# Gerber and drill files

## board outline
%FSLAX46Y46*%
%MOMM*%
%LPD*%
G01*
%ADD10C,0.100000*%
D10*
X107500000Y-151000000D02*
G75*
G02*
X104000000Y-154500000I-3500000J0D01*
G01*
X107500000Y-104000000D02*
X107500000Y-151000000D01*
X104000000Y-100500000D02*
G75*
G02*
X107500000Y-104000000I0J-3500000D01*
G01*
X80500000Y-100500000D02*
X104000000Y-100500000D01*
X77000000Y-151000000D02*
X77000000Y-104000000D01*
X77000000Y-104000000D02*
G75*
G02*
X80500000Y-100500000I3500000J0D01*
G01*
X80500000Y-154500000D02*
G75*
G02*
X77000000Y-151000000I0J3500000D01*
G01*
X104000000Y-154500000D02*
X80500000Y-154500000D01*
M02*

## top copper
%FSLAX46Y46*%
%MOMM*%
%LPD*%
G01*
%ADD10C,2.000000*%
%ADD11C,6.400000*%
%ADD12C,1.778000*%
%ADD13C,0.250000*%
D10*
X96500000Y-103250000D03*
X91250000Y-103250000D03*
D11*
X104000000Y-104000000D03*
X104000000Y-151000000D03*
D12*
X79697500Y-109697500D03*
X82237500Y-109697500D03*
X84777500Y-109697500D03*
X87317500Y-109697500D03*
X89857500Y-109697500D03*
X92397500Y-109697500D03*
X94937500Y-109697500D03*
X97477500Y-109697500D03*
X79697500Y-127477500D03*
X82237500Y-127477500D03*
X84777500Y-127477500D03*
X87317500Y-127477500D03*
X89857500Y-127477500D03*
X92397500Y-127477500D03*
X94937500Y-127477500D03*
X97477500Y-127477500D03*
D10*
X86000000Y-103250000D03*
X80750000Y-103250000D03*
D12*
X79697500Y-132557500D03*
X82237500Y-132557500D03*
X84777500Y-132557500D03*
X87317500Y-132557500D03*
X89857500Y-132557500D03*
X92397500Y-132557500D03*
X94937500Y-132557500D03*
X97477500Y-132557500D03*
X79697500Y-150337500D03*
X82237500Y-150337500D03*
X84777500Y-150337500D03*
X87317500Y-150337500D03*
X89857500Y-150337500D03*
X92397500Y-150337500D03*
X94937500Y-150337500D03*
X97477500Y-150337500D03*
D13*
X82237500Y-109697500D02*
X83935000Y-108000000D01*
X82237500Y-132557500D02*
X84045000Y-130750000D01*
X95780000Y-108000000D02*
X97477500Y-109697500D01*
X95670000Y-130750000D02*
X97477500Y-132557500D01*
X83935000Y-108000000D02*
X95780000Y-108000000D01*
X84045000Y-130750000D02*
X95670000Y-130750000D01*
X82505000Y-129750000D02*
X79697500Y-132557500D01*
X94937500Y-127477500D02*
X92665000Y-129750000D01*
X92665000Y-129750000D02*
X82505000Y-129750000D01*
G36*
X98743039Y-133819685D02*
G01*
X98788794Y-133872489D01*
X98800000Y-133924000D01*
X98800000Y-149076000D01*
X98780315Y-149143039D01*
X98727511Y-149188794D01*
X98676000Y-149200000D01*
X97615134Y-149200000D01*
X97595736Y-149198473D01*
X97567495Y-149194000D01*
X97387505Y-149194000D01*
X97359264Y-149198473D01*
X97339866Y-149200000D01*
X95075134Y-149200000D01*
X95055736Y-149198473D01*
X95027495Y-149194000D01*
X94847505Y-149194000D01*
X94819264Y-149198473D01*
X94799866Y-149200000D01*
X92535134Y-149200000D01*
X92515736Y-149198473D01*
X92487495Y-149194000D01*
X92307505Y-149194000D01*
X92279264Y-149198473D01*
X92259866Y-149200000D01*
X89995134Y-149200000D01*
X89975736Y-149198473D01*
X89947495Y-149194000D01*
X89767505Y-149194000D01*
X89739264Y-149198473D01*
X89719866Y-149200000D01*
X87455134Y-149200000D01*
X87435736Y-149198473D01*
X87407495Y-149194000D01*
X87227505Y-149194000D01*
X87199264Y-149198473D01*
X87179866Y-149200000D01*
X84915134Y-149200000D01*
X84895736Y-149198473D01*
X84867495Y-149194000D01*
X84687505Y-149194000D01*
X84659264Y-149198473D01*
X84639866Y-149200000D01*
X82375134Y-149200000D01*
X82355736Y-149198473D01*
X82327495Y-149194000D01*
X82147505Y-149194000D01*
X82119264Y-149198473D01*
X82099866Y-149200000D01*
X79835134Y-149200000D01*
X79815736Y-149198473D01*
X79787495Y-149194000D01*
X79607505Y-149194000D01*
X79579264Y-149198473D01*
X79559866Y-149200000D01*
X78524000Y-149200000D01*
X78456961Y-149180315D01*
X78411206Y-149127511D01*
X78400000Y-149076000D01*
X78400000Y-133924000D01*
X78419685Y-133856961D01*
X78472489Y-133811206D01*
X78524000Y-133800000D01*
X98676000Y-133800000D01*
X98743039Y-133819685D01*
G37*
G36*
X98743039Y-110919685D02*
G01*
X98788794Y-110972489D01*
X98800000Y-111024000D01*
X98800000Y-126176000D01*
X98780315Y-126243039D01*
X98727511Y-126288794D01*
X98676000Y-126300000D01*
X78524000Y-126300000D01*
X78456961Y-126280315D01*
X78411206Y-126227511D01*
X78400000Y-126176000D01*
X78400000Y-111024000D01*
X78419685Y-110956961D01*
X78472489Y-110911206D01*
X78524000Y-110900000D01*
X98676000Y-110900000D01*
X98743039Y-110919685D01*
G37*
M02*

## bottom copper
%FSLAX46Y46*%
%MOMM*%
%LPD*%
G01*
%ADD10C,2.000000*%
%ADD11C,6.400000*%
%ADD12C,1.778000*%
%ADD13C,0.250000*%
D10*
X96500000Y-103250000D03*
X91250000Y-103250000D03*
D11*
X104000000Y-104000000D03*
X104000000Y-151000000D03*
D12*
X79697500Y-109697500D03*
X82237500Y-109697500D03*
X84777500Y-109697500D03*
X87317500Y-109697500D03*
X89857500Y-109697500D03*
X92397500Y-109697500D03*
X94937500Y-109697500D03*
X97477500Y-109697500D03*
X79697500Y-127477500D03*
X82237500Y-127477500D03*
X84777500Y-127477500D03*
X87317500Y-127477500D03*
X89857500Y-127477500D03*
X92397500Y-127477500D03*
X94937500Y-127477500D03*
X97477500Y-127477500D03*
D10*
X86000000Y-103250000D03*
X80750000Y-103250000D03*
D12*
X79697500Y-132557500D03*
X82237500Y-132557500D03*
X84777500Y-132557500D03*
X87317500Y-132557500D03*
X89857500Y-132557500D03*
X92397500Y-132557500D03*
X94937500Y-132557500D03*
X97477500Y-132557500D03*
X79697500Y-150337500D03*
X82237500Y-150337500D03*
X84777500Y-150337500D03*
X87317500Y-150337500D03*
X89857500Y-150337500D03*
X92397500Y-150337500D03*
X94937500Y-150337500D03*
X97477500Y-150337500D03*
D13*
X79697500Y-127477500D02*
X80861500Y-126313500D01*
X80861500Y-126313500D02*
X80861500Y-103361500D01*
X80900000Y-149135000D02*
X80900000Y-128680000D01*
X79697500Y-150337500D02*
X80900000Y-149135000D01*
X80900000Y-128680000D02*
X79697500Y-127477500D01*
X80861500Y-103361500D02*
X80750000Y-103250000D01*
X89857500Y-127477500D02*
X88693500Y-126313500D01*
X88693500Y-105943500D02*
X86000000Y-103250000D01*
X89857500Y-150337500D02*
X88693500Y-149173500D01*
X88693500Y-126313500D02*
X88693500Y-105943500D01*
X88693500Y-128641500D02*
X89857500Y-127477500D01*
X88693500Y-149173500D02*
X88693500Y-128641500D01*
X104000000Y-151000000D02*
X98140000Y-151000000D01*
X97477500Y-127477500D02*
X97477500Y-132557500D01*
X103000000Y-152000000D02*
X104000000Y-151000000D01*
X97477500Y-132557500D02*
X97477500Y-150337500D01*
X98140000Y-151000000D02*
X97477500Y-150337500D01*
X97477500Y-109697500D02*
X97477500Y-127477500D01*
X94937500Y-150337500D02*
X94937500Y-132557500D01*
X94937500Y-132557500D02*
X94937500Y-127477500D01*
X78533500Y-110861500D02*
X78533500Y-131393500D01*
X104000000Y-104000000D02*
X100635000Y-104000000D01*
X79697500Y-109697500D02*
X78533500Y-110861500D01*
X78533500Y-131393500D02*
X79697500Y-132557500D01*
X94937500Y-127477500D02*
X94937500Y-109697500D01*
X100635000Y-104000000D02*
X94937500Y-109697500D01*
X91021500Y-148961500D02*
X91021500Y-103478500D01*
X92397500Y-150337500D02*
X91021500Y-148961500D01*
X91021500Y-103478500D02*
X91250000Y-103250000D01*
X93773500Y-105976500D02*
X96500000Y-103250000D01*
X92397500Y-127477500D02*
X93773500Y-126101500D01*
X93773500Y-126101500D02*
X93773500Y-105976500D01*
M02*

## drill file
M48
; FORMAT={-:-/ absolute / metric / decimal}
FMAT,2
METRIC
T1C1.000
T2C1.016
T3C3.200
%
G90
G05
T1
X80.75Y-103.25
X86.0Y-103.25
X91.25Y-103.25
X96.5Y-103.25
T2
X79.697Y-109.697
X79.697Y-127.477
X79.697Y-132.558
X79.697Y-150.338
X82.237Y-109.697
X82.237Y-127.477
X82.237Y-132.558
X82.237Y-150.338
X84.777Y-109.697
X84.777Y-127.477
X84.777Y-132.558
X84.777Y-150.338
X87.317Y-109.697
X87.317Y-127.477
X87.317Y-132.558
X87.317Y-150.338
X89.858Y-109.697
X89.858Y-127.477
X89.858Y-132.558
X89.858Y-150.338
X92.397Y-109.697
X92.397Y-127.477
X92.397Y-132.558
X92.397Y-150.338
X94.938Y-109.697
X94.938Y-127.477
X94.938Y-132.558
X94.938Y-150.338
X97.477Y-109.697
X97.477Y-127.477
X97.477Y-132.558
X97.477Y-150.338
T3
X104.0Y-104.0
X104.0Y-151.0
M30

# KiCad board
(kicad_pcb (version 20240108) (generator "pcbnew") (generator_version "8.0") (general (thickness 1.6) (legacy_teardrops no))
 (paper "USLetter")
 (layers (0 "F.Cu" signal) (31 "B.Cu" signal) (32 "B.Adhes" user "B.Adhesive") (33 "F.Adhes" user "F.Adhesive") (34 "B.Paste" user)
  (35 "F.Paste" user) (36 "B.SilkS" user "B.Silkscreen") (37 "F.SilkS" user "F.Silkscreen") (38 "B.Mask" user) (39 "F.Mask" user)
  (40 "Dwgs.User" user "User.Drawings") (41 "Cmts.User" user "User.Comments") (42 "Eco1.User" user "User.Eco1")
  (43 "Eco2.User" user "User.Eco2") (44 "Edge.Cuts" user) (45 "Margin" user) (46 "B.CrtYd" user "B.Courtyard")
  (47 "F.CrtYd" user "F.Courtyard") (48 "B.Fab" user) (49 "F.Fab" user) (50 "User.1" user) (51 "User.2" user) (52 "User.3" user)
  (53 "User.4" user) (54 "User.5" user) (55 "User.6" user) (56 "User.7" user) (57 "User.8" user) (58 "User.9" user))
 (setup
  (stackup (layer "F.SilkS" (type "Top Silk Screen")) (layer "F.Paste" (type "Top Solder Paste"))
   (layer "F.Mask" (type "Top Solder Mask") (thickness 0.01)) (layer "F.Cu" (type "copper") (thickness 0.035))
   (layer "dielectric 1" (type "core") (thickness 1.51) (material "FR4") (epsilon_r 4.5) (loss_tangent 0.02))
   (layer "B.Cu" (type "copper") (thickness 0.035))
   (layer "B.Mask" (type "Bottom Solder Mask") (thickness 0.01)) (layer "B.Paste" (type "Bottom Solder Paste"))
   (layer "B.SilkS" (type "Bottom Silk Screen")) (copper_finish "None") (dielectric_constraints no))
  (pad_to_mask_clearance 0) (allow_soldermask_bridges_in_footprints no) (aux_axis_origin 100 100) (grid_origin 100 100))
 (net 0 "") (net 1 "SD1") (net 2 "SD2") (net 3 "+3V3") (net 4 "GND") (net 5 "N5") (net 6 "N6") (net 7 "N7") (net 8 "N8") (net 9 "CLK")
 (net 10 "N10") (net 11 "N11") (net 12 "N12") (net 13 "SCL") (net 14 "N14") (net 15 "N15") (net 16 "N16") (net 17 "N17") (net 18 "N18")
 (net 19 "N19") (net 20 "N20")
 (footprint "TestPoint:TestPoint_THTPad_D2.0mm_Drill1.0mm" (layer "F.Cu") (at 96.5 103.25)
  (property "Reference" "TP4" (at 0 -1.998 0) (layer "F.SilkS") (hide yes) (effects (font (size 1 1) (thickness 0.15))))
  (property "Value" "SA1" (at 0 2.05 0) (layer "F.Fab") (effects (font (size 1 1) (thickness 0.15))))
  (pad "1" thru_hole circle (at 0 0) (size 2 2) (drill 1) (layers "*.Cu" "*.Mask") (remove_unused_layers no) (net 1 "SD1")))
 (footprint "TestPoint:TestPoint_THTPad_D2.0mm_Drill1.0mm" (layer "F.Cu") (at 91.25 103.25)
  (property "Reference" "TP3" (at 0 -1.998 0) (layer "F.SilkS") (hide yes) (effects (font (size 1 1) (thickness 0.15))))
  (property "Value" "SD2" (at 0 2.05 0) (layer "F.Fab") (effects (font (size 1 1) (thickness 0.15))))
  (pad "1" thru_hole circle (at 0 0) (size 2 2) (drill 1) (layers "*.Cu" "*.Mask") (remove_unused_layers no) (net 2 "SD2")))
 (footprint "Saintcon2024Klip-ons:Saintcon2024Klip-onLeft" (layer "F.Cu") (at 139.75 126.4)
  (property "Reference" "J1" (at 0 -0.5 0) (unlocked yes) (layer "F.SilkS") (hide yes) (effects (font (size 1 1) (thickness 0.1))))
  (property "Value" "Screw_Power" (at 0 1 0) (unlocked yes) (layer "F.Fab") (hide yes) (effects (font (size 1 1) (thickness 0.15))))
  (pad "+" thru_hole circle (at -35.75 -22.4) (size 6.4 6.4) (drill 3.2) (layers "*.Cu" "*.Mask") (remove_unused_layers no) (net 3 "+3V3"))
  (pad "-" thru_hole circle (at -35.75 24.6) (size 6.4 6.4) (drill 3.2) (layers "*.Cu" "*.Mask") (remove_unused_layers no) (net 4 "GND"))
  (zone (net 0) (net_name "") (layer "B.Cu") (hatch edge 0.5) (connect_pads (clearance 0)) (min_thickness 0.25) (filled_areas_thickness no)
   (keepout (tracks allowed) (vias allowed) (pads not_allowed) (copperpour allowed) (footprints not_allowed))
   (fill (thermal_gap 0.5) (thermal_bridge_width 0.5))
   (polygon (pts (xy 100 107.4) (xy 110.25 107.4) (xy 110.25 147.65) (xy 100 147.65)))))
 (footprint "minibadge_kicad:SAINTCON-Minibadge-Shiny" (layer "F.Cu") (at 78.4275 108.4275)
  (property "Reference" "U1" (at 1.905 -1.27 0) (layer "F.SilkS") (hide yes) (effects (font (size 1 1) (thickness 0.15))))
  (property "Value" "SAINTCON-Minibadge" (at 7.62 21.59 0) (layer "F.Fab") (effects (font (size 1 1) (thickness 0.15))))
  (pad "1" thru_hole circle (at 1.27 1.27 90) (size 1.778 1.778) (drill 1.016) (layers "*.Cu" "*.Mask") (remove_unused_layers no)
   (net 3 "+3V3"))
  (pad "2" thru_hole circle (at 3.81 1.27 90) (size 1.778 1.778) (drill 1.016) (layers "*.Cu" "*.Mask") (remove_unused_layers no)
   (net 4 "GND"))
  (pad "3" thru_hole circle (at 6.35 1.27 90) (size 1.778 1.778) (drill 1.016) (layers "*.Cu" "*.Mask") (remove_unused_layers no)
   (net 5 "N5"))
  (pad "4" thru_hole circle (at 8.89 1.27 90) (size 1.778 1.778) (drill 1.016) (layers "*.Cu" "*.Mask") (remove_unused_layers no)
   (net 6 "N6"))
  (pad "5" thru_hole circle (at 11.43 1.27 90) (size 1.778 1.778) (drill 1.016) (layers "*.Cu" "*.Mask") (remove_unused_layers no)
   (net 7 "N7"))
  (pad "6" thru_hole circle (at 13.97 1.27 90) (size 1.778 1.778) (drill 1.016) (layers "*.Cu" "*.Mask") (remove_unused_layers no)
   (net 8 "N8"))
  (pad "7" thru_hole circle (at 16.51 1.27 90) (size 1.778 1.778) (drill 1.016) (layers "*.Cu" "*.Mask") (remove_unused_layers no)
   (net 3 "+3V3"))
  (pad "8" thru_hole circle (at 19.05 1.27 90) (size 1.778 1.778) (drill 1.016) (layers "*.Cu" "*.Mask") (remove_unused_layers no)
   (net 4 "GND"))
  (pad "9" thru_hole circle (at 1.27 19.05 90) (size 1.778 1.778) (drill 1.016) (layers "*.Cu" "*.Mask") (remove_unused_layers no)
   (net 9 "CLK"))
  (pad "10" thru_hole circle (at 3.81 19.05 90) (size 1.778 1.778) (drill 1.016) (layers "*.Cu" "*.Mask") (remove_unused_layers no)
   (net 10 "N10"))
  (pad "11" thru_hole circle (at 6.35 19.05 90) (size 1.778 1.778) (drill 1.016) (layers "*.Cu" "*.Mask") (remove_unused_layers no)
   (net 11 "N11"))
  (pad "12" thru_hole circle (at 8.89 19.05 90) (size 1.778 1.778) (drill 1.016) (layers "*.Cu" "*.Mask") (remove_unused_layers no)
   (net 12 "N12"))
  (pad "13" thru_hole circle (at 11.43 19.05 90) (size 1.778 1.778) (drill 1.016) (layers "*.Cu" "*.Mask") (remove_unused_layers no)
   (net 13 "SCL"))
  (pad "14" thru_hole circle (at 13.97 19.05 90) (size 1.778 1.778) (drill 1.016) (layers "*.Cu" "*.Mask") (remove_unused_layers no)
   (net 1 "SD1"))
  (pad "15" thru_hole circle (at 16.51 19.05 90) (size 1.778 1.778) (drill 1.016) (layers "*.Cu" "*.Mask") (remove_unused_layers no)
   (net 3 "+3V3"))
  (pad "16" thru_hole circle (at 19.05 19.05 90) (size 1.778 1.778) (drill 1.016) (layers "*.Cu" "*.Mask") (remove_unused_layers no)
   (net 4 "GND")))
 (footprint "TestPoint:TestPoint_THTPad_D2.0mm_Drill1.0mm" (layer "F.Cu") (at 86 103.25)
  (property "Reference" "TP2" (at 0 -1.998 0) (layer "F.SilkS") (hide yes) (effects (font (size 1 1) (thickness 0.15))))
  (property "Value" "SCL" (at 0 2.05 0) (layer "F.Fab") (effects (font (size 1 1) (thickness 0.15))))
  (pad "1" thru_hole circle (at 0 0) (size 2 2) (drill 1) (layers "*.Cu" "*.Mask") (remove_unused_layers no) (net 13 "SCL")))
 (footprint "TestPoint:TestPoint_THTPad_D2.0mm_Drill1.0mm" (layer "F.Cu") (at 80.75 103.25)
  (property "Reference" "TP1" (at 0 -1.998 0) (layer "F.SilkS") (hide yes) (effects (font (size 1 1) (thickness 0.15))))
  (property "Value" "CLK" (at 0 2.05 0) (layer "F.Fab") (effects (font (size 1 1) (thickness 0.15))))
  (pad "1" thru_hole circle (at 0 0) (size 2 2) (drill 1) (layers "*.Cu" "*.Mask") (remove_unused_layers no) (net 9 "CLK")))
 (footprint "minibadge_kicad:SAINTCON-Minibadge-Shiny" (layer "F.Cu") (at 78.4275 131.2875)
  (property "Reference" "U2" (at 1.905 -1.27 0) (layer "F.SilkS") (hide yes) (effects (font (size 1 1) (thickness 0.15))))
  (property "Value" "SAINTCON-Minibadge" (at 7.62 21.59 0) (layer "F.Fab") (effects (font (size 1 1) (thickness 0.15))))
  (pad "1" thru_hole circle (at 1.27 1.27 90) (size 1.778 1.778) (drill 1.016) (layers "*.Cu" "*.Mask") (remove_unused_layers no)
   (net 3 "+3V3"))
  (pad "2" thru_hole circle (at 3.81 1.27 90) (size 1.778 1.778) (drill 1.016) (layers "*.Cu" "*.Mask") (remove_unused_layers no)
   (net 4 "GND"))
  (pad "3" thru_hole circle (at 6.35 1.27 90) (size 1.778 1.778) (drill 1.016) (layers "*.Cu" "*.Mask") (remove_unused_layers no)
   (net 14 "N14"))
  (pad "4" thru_hole circle (at 8.89 1.27 90) (size 1.778 1.778) (drill 1.016) (layers "*.Cu" "*.Mask") (remove_unused_layers no)
   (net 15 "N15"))
  (pad "5" thru_hole circle (at 11.43 1.27 90) (size 1.778 1.778) (drill 1.016) (layers "*.Cu" "*.Mask") (remove_unused_layers no)
   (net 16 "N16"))
  (pad "6" thru_hole circle (at 13.97 1.27 90) (size 1.778 1.778) (drill 1.016) (layers "*.Cu" "*.Mask") (remove_unused_layers no)
   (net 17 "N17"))
  (pad "7" thru_hole circle (at 16.51 1.27 90) (size 1.778 1.778) (drill 1.016) (layers "*.Cu" "*.Mask") (remove_unused_layers no)
   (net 3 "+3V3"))
  (pad "8" thru_hole circle (at 19.05 1.27 90) (size 1.778 1.778) (drill 1.016) (layers "*.Cu" "*.Mask") (remove_unused_layers no)
   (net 4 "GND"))
  (pad "9" thru_hole circle (at 1.27 19.05 90) (size 1.778 1.778) (drill 1.016) (layers "*.Cu" "*.Mask") (remove_unused_layers no)
   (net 9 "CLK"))
  (pad "10" thru_hole circle (at 3.81 19.05 90) (size 1.778 1.778) (drill 1.016) (layers "*.Cu" "*.Mask") (remove_unused_layers no)
   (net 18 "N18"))
  (pad "11" thru_hole circle (at 6.35 19.05 90) (size 1.778 1.778) (drill 1.016) (layers "*.Cu" "*.Mask") (remove_unused_layers no)
   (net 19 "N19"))
  (pad "12" thru_hole circle (at 8.89 19.05 90) (size 1.778 1.778) (drill 1.016) (layers "*.Cu" "*.Mask") (remove_unused_layers no)
   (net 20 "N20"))
  (pad "13" thru_hole circle (at 11.43 19.05 90) (size 1.778 1.778) (drill 1.016) (layers "*.Cu" "*.Mask") (remove_unused_layers no)
   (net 13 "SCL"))
  (pad "14" thru_hole circle (at 13.97 19.05 90) (size 1.778 1.778) (drill 1.016) (layers "*.Cu" "*.Mask") (remove_unused_layers no)
   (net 2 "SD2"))
  (pad "15" thru_hole circle (at 16.51 19.05 90) (size 1.778 1.778) (drill 1.016) (layers "*.Cu" "*.Mask") (remove_unused_layers no)
   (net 3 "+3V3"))
  (pad "16" thru_hole circle (at 19.05 19.05 90) (size 1.778 1.778) (drill 1.016) (layers "*.Cu" "*.Mask") (remove_unused_layers no)
   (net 4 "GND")))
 (gr_arc (start 107.5 151) (mid 106.474874 153.474874) (end 104 154.5) (stroke (width 0.1) (type default)) (layer "Edge.Cuts"))
 (gr_line (start 107.5 104) (end 107.5 151) (stroke (width 0.1) (type default)) (layer "Edge.Cuts"))
 (gr_arc (start 104 100.5) (mid 106.474874 101.525126) (end 107.5 104) (stroke (width 0.1) (type default)) (layer "Edge.Cuts"))
 (gr_line (start 80.5 100.5) (end 104 100.5) (stroke (width 0.1) (type default)) (layer "Edge.Cuts"))
 (gr_line (start 77 151) (end 77 104) (stroke (width 0.1) (type default)) (layer "Edge.Cuts"))
 (gr_arc (start 77 104) (mid 78.025126 101.525126) (end 80.5 100.5) (stroke (width 0.1) (type default)) (layer "Edge.Cuts"))
 (gr_arc (start 80.5 154.5) (mid 78.025126 153.474874) (end 77 151) (stroke (width 0.1) (type default)) (layer "Edge.Cuts"))
 (gr_line (start 104 154.5) (end 80.5 154.5) (stroke (width 0.1) (type default)) (layer "Edge.Cuts"))
 (segment (start 79.6975 127.4775) (end 80.8615 126.3135) (width 0.25) (layer "B.Cu") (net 9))
 (segment (start 80.8615 126.3135) (end 80.8615 103.3615) (width 0.25) (layer "B.Cu") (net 9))
 (segment (start 80.9 149.135) (end 80.9 128.68) (width 0.25) (layer "B.Cu") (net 9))
 (segment (start 79.6975 150.3375) (end 80.9 149.135) (width 0.25) (layer "B.Cu") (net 9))
 (segment (start 80.9 128.68) (end 79.6975 127.4775) (width 0.25) (layer "B.Cu") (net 9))
 (segment (start 80.8615 103.3615) (end 80.75 103.25) (width 0.25) (layer "B.Cu") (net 9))
 (segment (start 89.8575 127.4775) (end 88.6935 126.3135) (width 0.25) (layer "B.Cu") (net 13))
 (segment (start 88.6935 105.9435) (end 86 103.25) (width 0.25) (layer "B.Cu") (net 13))
 (segment (start 89.8575 150.3375) (end 88.6935 149.1735) (width 0.25) (layer "B.Cu") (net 13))
 (segment (start 88.6935 126.3135) (end 88.6935 105.9435) (width 0.25) (layer "B.Cu") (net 13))
 (segment (start 88.6935 128.6415) (end 89.8575 127.4775) (width 0.25) (layer "B.Cu") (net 13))
 (segment (start 88.6935 149.1735) (end 88.6935 128.6415) (width 0.25) (layer "B.Cu") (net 13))
 (segment (start 82.2375 109.6975) (end 83.935 108) (width 0.25) (layer "F.Cu") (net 4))
 (segment (start 82.2375 132.5575) (end 84.045 130.75) (width 0.25) (layer "F.Cu") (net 4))
 (segment (start 95.78 108) (end 97.4775 109.6975) (width 0.25) (layer "F.Cu") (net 4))
 (segment (start 95.67 130.75) (end 97.4775 132.5575) (width 0.25) (layer "F.Cu") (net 4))
 (segment (start 83.935 108) (end 95.78 108) (width 0.25) (layer "F.Cu") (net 4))
 (segment (start 84.045 130.75) (end 95.67 130.75) (width 0.25) (layer "F.Cu") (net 4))
 (segment (start 104 151) (end 98.14 151) (width 0.25) (layer "B.Cu") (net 4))
 (segment (start 97.4775 127.4775) (end 97.4775 132.5575) (width 0.25) (layer "B.Cu") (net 4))
 (segment (start 103 152) (end 104 151) (width 0.25) (layer "B.Cu") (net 4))
 (segment (start 97.4775 132.5575) (end 97.4775 150.3375) (width 0.25) (layer "B.Cu") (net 4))
 (segment (start 98.14 151) (end 97.4775 150.3375) (width 0.25) (layer "B.Cu") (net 4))
 (segment (start 97.4775 109.6975) (end 97.4775 127.4775) (width 0.25) (layer "B.Cu") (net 4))
 (segment (start 82.505 129.75) (end 79.6975 132.5575) (width 0.25) (layer "F.Cu") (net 3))
 (segment (start 94.9375 127.4775) (end 92.665 129.75) (width 0.25) (layer "F.Cu") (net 3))
 (segment (start 92.665 129.75) (end 82.505 129.75) (width 0.25) (layer "F.Cu") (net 3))
 (segment (start 94.9375 150.3375) (end 94.9375 132.5575) (width 0.25) (layer "B.Cu") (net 3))
 (segment (start 94.9375 132.5575) (end 94.9375 127.4775) (width 0.25) (layer "B.Cu") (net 3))
 (segment (start 78.5335 110.8615) (end 78.5335 131.3935) (width 0.25) (layer "B.Cu") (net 3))
 (segment (start 104 104) (end 100.635 104) (width 0.25) (layer "B.Cu") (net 3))
 (segment (start 79.6975 109.6975) (end 78.5335 110.8615) (width 0.25) (layer "B.Cu") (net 3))
 (segment (start 78.5335 131.3935) (end 79.6975 132.5575) (width 0.25) (layer "B.Cu") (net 3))
 (segment (start 94.9375 127.4775) (end 94.9375 109.6975) (width 0.25) (layer "B.Cu") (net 3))
 (segment (start 100.635 104) (end 94.9375 109.6975) (width 0.25) (layer "B.Cu") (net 3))
 (segment (start 91.0215 148.9615) (end 91.0215 103.4785) (width 0.25) (layer "B.Cu") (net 2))
 (segment (start 92.3975 150.3375) (end 91.0215 148.9615) (width 0.25) (layer "B.Cu") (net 2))
 (segment (start 91.0215 103.4785) (end 91.25 103.25) (width 0.25) (layer "B.Cu") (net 2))
 (segment (start 93.7735 105.9765) (end 96.5 103.25) (width 0.25) (layer "B.Cu") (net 1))
 (segment (start 92.3975 127.4775) (end 93.7735 126.1015) (width 0.25) (layer "B.Cu") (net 1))
 (segment (start 93.7735 126.1015) (end 93.7735 105.9765) (width 0.25) (layer "B.Cu") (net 1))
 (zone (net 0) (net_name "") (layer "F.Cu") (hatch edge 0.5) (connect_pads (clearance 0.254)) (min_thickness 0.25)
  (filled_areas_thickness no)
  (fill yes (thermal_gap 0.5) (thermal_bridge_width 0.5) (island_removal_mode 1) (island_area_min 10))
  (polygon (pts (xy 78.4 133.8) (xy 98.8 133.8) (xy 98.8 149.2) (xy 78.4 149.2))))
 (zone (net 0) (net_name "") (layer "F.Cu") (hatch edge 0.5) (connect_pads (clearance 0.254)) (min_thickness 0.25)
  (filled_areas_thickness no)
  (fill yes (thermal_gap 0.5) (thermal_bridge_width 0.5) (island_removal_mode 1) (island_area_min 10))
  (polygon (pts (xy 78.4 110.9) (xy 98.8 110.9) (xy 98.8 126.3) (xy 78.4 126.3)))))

